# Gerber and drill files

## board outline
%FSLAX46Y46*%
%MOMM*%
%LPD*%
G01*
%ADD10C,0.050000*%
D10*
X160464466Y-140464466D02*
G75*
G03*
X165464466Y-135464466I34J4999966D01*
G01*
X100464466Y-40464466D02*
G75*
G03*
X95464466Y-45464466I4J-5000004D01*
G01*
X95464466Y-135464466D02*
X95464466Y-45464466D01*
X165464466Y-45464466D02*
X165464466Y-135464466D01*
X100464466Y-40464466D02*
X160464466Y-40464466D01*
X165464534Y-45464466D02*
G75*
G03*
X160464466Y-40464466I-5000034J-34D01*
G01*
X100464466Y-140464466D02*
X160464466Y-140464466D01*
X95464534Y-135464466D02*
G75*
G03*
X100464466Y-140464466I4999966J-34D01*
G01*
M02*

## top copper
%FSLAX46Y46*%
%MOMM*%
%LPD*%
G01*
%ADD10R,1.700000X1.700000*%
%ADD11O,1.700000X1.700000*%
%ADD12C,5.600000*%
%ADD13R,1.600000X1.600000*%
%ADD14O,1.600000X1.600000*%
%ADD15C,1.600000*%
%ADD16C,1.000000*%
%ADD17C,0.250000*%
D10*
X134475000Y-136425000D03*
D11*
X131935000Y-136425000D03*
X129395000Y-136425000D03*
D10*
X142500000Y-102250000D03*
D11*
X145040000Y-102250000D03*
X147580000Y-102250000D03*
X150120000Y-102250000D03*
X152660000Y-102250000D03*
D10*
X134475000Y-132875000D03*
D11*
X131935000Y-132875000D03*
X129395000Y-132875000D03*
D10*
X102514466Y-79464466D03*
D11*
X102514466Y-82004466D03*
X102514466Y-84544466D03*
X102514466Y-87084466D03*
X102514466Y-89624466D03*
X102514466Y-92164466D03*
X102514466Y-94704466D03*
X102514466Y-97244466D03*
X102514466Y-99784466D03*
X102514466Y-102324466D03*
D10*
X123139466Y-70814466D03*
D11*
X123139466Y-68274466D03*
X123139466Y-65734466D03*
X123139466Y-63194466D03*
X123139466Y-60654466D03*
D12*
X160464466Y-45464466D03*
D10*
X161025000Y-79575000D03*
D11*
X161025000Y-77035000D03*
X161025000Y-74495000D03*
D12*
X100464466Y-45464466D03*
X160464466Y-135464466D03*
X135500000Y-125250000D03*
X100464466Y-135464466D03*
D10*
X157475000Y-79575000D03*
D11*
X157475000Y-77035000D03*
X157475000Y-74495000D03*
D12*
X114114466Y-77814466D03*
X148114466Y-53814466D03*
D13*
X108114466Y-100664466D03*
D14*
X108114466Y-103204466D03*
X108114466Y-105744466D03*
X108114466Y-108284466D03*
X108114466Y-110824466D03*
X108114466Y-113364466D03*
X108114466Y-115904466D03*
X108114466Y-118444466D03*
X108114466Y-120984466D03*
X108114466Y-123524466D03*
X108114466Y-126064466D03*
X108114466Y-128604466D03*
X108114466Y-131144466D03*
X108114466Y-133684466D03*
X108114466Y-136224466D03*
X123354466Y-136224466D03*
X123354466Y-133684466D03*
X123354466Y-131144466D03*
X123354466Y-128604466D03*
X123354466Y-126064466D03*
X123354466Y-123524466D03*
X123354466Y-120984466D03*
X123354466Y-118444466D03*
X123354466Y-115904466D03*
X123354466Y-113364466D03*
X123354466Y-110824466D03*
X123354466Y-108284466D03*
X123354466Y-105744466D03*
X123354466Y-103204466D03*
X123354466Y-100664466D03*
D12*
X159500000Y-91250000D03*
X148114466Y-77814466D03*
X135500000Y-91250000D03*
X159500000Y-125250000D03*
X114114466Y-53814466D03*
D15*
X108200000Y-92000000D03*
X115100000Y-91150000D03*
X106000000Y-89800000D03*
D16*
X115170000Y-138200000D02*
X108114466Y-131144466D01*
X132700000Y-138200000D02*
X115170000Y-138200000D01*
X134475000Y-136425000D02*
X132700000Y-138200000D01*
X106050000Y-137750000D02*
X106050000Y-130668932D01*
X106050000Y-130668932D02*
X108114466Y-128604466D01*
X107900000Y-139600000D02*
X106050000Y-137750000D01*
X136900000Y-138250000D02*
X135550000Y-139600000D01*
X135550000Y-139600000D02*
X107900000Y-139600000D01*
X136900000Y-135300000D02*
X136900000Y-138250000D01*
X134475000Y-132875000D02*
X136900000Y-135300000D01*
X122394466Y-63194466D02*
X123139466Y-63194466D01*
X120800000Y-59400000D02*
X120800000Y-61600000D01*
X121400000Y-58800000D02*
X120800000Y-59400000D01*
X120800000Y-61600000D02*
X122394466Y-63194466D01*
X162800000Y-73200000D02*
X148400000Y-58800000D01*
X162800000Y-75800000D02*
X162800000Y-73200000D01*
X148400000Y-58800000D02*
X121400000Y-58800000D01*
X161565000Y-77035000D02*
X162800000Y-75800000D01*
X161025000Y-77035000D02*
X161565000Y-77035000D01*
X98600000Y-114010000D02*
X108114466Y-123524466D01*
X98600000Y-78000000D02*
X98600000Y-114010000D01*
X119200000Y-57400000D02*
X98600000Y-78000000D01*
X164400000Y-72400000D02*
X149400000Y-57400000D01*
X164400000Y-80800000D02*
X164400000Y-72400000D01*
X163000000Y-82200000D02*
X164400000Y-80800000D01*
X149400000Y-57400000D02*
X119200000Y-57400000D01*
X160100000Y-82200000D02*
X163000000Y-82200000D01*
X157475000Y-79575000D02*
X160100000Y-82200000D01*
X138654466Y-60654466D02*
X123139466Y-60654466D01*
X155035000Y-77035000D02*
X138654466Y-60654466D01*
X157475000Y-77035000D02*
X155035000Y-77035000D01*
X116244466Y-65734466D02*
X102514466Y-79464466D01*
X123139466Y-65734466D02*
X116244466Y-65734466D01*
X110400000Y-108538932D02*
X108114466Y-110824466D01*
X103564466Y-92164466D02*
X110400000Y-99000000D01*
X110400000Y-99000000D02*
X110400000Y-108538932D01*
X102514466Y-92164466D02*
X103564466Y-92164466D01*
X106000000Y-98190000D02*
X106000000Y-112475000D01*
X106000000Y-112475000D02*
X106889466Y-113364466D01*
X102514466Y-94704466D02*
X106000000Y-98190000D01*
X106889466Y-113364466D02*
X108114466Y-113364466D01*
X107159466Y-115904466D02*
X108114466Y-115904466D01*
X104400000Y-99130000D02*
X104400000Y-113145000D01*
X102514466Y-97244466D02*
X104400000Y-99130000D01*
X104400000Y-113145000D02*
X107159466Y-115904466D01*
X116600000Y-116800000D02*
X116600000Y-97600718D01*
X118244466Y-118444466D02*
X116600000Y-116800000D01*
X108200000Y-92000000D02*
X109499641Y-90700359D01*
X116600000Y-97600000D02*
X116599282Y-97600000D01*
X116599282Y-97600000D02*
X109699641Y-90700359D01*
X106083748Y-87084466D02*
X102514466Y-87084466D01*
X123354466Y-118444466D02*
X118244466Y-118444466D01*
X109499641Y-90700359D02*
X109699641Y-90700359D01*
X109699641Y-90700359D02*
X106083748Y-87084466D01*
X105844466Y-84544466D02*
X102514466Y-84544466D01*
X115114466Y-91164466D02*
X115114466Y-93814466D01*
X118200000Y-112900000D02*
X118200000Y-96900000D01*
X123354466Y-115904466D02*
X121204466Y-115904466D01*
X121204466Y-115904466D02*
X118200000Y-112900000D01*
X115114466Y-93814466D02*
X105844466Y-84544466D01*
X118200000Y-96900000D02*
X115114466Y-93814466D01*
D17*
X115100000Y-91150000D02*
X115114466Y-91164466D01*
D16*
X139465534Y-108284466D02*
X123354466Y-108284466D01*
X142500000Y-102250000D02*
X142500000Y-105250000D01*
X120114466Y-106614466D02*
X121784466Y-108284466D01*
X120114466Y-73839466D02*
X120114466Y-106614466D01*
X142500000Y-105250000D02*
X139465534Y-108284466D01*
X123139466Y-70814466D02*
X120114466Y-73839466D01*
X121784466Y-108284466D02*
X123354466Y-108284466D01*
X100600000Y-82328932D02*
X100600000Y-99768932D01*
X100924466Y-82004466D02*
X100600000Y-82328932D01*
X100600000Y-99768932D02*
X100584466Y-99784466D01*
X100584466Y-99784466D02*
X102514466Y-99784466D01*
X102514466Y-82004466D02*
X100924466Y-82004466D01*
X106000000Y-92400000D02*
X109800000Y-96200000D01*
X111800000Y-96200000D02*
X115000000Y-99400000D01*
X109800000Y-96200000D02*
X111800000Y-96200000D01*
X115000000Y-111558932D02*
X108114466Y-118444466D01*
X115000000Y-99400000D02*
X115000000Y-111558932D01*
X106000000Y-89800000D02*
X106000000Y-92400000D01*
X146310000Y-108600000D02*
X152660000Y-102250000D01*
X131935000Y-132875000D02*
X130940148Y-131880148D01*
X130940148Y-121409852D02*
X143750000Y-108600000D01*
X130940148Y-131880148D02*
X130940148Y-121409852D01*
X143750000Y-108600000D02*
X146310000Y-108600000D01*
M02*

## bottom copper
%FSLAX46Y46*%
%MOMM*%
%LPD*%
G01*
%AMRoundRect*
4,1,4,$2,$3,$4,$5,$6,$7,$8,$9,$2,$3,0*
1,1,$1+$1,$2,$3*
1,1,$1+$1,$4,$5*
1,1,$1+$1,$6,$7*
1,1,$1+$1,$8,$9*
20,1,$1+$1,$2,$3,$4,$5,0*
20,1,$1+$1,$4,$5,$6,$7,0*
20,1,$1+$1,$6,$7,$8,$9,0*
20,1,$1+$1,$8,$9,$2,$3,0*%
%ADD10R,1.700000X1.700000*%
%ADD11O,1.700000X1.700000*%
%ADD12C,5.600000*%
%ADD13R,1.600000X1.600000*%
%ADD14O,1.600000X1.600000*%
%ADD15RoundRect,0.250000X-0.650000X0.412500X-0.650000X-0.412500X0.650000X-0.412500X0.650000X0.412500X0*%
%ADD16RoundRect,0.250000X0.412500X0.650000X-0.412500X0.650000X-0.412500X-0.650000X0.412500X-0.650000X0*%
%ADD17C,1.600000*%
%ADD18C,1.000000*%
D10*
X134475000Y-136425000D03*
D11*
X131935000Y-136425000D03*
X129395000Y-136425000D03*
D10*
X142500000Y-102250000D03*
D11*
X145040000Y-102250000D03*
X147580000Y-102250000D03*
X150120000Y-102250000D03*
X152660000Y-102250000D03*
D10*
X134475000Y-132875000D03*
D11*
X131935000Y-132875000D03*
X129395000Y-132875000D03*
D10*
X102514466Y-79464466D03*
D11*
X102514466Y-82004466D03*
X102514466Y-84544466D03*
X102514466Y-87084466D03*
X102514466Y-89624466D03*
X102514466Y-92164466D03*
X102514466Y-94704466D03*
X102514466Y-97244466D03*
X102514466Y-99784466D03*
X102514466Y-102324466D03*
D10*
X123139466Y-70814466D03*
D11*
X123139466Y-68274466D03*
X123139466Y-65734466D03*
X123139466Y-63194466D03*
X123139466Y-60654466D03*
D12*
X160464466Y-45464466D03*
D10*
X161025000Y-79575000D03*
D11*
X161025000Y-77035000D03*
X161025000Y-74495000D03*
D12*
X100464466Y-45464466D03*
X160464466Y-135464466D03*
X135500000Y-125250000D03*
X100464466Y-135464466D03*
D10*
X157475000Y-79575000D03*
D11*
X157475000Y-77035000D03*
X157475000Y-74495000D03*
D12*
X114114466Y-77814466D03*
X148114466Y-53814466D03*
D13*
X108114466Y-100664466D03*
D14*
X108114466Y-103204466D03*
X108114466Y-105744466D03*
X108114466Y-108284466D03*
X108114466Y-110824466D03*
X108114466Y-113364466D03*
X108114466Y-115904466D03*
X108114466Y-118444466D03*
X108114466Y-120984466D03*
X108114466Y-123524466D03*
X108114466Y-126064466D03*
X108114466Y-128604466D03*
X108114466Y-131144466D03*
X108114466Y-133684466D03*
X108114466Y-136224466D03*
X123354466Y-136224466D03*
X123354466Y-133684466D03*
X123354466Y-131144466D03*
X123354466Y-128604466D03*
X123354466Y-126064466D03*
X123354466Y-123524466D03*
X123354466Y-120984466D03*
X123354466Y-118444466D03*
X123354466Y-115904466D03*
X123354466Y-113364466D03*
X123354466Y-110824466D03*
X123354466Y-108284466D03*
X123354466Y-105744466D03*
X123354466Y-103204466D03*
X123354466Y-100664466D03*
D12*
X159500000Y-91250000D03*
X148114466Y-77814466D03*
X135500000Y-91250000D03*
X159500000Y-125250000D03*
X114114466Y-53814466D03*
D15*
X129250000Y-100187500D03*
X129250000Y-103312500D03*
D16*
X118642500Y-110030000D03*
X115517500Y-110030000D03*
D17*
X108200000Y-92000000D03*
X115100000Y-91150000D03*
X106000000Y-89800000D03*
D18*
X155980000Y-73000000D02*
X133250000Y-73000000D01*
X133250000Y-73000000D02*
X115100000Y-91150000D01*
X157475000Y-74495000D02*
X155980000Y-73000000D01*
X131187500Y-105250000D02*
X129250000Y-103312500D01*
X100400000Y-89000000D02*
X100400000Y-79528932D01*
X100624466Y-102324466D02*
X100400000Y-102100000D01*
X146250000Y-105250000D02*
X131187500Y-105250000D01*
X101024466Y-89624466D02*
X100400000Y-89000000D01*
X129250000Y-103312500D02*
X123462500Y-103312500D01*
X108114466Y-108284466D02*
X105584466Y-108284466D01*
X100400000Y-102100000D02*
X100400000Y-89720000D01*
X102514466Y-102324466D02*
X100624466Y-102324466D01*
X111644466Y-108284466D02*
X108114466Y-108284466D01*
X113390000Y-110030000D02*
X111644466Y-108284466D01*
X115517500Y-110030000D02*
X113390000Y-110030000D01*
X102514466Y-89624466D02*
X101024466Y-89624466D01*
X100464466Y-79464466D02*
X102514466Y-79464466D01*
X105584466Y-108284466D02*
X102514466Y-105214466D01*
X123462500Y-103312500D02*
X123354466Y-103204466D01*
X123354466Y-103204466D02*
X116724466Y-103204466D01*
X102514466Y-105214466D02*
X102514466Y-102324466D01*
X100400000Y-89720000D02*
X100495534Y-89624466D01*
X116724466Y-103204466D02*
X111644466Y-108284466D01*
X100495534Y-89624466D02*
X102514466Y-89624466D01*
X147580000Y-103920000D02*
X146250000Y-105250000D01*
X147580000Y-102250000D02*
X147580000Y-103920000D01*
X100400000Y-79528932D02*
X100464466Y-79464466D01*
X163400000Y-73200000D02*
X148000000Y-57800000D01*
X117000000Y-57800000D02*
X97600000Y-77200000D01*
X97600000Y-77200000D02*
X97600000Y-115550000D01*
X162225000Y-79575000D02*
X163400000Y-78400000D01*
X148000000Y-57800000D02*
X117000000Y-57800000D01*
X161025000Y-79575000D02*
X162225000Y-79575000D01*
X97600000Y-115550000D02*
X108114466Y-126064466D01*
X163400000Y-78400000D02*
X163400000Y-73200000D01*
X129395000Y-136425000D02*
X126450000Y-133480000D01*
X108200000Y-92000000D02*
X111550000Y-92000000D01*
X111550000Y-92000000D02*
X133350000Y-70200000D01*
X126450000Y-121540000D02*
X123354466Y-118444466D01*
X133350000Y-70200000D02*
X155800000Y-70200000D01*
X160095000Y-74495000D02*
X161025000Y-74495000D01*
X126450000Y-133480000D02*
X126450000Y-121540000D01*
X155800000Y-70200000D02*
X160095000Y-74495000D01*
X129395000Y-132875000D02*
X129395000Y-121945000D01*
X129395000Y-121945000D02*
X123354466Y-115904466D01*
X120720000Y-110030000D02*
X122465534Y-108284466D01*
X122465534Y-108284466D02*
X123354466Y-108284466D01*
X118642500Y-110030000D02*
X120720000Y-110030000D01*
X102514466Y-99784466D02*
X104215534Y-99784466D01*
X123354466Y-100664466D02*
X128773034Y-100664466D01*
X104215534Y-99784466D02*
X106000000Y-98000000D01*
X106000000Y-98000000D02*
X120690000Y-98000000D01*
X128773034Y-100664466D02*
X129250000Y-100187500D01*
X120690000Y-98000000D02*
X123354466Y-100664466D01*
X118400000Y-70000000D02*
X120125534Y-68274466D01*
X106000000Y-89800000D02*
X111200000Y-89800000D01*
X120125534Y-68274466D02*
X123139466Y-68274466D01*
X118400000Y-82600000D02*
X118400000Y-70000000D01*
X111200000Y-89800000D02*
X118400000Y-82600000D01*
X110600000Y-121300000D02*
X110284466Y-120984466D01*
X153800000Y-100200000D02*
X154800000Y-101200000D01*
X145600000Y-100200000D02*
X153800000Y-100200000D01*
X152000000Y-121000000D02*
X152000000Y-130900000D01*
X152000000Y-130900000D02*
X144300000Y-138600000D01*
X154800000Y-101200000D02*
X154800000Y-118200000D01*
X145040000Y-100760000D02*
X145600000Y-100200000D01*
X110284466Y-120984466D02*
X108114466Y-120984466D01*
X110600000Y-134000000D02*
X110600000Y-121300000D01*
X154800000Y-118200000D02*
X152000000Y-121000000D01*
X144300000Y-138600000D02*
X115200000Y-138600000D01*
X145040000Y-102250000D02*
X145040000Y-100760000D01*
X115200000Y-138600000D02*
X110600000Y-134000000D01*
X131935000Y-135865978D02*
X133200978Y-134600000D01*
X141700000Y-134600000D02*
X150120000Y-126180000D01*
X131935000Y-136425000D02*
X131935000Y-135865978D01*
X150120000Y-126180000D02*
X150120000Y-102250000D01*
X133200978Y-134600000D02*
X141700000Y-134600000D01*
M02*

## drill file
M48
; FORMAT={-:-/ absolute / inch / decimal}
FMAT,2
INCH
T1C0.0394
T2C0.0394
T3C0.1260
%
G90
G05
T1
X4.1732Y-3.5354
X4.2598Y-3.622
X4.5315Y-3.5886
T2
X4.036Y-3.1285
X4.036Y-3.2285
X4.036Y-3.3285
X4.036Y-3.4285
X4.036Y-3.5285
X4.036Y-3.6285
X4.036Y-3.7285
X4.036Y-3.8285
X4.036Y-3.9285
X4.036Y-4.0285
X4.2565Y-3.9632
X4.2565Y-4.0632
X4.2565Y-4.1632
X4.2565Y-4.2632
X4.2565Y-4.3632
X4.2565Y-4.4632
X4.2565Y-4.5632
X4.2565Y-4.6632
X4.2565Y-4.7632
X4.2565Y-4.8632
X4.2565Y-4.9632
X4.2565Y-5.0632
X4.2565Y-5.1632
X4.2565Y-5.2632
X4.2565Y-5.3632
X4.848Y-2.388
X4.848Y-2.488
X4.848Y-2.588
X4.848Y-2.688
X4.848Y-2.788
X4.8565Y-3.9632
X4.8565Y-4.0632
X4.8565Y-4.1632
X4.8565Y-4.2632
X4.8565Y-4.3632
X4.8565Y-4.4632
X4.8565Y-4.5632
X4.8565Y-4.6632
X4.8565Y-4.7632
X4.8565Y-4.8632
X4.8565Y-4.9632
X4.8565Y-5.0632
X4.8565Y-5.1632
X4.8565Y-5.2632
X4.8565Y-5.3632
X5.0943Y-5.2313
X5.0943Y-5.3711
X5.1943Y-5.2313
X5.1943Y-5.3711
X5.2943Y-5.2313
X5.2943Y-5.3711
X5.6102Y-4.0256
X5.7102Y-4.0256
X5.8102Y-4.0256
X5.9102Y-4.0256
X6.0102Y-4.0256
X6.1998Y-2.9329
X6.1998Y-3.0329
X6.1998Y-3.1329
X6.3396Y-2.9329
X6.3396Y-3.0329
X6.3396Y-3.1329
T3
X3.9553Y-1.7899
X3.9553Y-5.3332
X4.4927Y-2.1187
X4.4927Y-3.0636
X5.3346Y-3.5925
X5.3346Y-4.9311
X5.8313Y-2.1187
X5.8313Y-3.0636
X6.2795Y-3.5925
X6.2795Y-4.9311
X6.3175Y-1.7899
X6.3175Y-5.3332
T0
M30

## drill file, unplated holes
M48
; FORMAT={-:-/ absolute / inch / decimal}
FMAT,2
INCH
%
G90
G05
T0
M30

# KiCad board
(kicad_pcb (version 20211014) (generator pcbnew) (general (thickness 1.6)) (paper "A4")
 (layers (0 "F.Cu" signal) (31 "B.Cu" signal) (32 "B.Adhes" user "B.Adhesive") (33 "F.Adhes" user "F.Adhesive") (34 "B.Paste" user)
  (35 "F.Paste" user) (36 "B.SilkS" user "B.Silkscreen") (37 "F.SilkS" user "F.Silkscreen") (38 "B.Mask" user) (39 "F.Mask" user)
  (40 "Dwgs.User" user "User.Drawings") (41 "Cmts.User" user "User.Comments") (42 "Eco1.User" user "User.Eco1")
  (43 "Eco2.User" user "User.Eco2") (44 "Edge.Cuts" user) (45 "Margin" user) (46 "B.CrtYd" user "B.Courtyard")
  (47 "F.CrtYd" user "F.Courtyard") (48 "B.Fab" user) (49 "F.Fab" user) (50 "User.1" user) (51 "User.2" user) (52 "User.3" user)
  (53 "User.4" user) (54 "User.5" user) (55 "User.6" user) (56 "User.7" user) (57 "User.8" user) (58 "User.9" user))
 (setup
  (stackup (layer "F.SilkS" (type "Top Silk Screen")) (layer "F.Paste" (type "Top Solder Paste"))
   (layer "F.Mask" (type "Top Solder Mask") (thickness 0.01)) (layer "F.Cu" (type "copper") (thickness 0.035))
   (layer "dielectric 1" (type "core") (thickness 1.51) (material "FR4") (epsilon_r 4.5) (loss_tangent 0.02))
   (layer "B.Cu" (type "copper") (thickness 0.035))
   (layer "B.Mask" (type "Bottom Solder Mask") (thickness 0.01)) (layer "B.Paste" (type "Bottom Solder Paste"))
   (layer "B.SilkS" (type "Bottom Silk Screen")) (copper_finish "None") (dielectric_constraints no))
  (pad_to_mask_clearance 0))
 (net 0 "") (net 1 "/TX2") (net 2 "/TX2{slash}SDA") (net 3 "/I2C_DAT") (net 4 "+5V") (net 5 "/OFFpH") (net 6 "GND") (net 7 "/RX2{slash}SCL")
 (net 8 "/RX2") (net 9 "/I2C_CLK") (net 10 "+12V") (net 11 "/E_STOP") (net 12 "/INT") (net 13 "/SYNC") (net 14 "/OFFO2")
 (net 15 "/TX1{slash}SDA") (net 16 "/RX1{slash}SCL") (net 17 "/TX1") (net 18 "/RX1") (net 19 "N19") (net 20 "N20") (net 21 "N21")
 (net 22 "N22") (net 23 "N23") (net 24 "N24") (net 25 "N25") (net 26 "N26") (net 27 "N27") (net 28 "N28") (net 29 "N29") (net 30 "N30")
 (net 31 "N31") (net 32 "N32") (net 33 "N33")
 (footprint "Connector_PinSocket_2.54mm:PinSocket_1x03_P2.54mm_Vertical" (layer "F.Cu") (at 134.475 136.425 -90)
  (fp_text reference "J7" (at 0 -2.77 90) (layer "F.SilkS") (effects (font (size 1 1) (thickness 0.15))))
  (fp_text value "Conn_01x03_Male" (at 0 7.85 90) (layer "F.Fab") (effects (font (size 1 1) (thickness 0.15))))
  (pad "1" thru_hole rect (at 0 0 270) (size 1.7 1.7) (drill 1) (layers *.Cu *.Mask) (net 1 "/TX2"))
  (pad "2" thru_hole oval (at 0 2.54 270) (size 1.7 1.7) (drill 1) (layers *.Cu *.Mask) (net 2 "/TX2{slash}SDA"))
  (pad "3" thru_hole oval (at 0 5.08 270) (size 1.7 1.7) (drill 1) (layers *.Cu *.Mask) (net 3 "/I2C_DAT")))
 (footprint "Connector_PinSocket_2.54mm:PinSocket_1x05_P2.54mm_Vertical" (layer "F.Cu") (at 142.5 102.25 90)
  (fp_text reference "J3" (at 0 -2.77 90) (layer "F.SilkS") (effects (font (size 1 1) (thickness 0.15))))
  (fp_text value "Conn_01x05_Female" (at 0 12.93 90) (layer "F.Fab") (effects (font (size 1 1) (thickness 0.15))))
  (pad "1" thru_hole rect (at 0 0 90) (size 1.7 1.7) (drill 1) (layers *.Cu *.Mask) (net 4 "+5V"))
  (pad "2" thru_hole oval (at 0 2.54 90) (size 1.7 1.7) (drill 1) (layers *.Cu *.Mask) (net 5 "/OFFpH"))
  (pad "3" thru_hole oval (at 0 5.08 90) (size 1.7 1.7) (drill 1) (layers *.Cu *.Mask) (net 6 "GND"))
  (pad "4" thru_hole oval (at 0 7.62 90) (size 1.7 1.7) (drill 1) (layers *.Cu *.Mask) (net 2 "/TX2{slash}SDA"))
  (pad "5" thru_hole oval (at 0 10.16 90) (size 1.7 1.7) (drill 1) (layers *.Cu *.Mask) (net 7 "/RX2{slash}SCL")))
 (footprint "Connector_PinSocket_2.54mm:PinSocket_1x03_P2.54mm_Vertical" (layer "F.Cu") (at 134.475 132.875 -90)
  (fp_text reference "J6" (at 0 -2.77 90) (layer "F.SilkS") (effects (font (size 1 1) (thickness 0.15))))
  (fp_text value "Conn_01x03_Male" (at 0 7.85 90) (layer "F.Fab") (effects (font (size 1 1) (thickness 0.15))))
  (pad "1" thru_hole rect (at 0 0 270) (size 1.7 1.7) (drill 1) (layers *.Cu *.Mask) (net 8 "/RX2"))
  (pad "2" thru_hole oval (at 0 2.54 270) (size 1.7 1.7) (drill 1) (layers *.Cu *.Mask) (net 7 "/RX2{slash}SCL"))
  (pad "3" thru_hole oval (at 0 5.08 270) (size 1.7 1.7) (drill 1) (layers *.Cu *.Mask) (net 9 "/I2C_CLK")))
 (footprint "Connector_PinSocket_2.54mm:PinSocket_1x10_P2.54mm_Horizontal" (layer "F.Cu") (at 102.514466 79.464466)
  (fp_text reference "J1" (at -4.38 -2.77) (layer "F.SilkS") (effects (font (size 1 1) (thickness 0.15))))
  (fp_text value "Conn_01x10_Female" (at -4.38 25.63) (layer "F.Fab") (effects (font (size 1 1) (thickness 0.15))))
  (pad "1" thru_hole rect (at 0 0) (size 1.7 1.7) (drill 1) (layers *.Cu *.Mask) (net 6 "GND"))
  (pad "2" thru_hole oval (at 0 2.54) (size 1.7 1.7) (drill 1) (layers *.Cu *.Mask) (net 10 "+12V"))
  (pad "3" thru_hole oval (at 0 5.08) (size 1.7 1.7) (drill 1) (layers *.Cu *.Mask) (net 9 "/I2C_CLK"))
  (pad "4" thru_hole oval (at 0 7.62) (size 1.7 1.7) (drill 1) (layers *.Cu *.Mask) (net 3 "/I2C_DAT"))
  (pad "5" thru_hole oval (at 0 10.16) (size 1.7 1.7) (drill 1) (layers *.Cu *.Mask) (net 6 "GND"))
  (pad "6" thru_hole oval (at 0 12.7) (size 1.7 1.7) (drill 1) (layers *.Cu *.Mask) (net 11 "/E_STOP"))
  (pad "7" thru_hole oval (at 0 15.24) (size 1.7 1.7) (drill 1) (layers *.Cu *.Mask) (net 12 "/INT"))
  (pad "8" thru_hole oval (at 0 17.78) (size 1.7 1.7) (drill 1) (layers *.Cu *.Mask) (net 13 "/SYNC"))
  (pad "9" thru_hole oval (at 0 20.32) (size 1.7 1.7) (drill 1) (layers *.Cu *.Mask) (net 10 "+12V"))
  (pad "10" thru_hole oval (at 0 22.86) (size 1.7 1.7) (drill 1) (layers *.Cu *.Mask) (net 6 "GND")))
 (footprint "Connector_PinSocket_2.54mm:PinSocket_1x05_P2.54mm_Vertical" (layer "F.Cu") (at 123.139466 70.814466 180)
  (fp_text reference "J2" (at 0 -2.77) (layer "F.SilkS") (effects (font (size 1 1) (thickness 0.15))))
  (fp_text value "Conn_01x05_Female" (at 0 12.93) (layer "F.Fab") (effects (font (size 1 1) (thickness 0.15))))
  (pad "1" thru_hole rect (at 0 0 180) (size 1.7 1.7) (drill 1) (layers *.Cu *.Mask) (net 4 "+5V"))
  (pad "2" thru_hole oval (at 0 2.54 180) (size 1.7 1.7) (drill 1) (layers *.Cu *.Mask) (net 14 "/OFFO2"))
  (pad "3" thru_hole oval (at 0 5.08 180) (size 1.7 1.7) (drill 1) (layers *.Cu *.Mask) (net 6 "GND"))
  (pad "4" thru_hole oval (at 0 7.62 180) (size 1.7 1.7) (drill 1) (layers *.Cu *.Mask) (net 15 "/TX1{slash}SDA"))
  (pad "5" thru_hole oval (at 0 10.16 180) (size 1.7 1.7) (drill 1) (layers *.Cu *.Mask) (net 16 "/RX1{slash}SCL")))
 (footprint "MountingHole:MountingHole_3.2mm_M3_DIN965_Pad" (layer "F.Cu") (at 160.464466 45.464466)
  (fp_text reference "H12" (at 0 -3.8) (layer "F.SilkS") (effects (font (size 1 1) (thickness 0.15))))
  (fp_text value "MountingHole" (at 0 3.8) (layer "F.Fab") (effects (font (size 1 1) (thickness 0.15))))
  (pad "1" thru_hole circle (at 0 0) (size 5.6 5.6) (drill 3.2) (layers *.Cu *.Mask)))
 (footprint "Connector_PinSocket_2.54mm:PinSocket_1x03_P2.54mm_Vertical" (layer "F.Cu") (at 161.025 79.575 180)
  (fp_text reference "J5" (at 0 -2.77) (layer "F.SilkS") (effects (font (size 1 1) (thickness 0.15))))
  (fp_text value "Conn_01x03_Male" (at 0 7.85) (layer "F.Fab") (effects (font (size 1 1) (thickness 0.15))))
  (pad "1" thru_hole rect (at 0 0 180) (size 1.7 1.7) (drill 1) (layers *.Cu *.Mask) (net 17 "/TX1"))
  (pad "2" thru_hole oval (at 0 2.54 180) (size 1.7 1.7) (drill 1) (layers *.Cu *.Mask) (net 15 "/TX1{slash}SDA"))
  (pad "3" thru_hole oval (at 0 5.08 180) (size 1.7 1.7) (drill 1) (layers *.Cu *.Mask) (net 3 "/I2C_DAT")))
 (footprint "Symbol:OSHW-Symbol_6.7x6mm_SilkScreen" (layer "F.Cu") (at 109.515 44.979 180)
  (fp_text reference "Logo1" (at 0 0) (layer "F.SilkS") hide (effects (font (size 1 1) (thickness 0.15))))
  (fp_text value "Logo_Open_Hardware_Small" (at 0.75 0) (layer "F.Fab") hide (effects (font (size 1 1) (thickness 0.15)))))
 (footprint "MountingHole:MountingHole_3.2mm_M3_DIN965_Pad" (layer "F.Cu") (at 100.464466 45.464466)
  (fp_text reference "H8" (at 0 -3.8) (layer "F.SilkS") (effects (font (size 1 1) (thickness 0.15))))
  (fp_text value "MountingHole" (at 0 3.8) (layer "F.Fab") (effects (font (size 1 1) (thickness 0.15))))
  (pad "1" thru_hole circle (at 0 0) (size 5.6 5.6) (drill 3.2) (layers *.Cu *.Mask)))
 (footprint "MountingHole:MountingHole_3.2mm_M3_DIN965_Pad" (layer "F.Cu") (at 160.464466 135.464466)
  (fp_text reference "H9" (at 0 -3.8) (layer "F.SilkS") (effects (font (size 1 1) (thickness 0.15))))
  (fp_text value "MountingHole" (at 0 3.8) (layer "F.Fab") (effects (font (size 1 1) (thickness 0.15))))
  (pad "1" thru_hole circle (at 0 0) (size 5.6 5.6) (drill 3.2) (layers *.Cu *.Mask)))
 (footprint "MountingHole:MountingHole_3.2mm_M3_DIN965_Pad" (layer "F.Cu") (at 135.5 125.25 90)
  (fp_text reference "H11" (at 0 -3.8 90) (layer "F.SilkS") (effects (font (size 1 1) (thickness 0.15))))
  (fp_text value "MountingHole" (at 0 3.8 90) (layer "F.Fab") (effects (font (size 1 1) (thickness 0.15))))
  (pad "1" thru_hole circle (at 0 0 90) (size 5.6 5.6) (drill 3.2) (layers *.Cu *.Mask)))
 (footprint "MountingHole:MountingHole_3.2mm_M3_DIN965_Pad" (layer "F.Cu") (at 100.464466 135.464466)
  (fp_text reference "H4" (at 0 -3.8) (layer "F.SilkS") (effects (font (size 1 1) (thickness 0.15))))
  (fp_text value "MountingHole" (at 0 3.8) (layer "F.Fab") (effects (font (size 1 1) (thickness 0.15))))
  (pad "1" thru_hole circle (at 0 0) (size 5.6 5.6) (drill 3.2) (layers *.Cu *.Mask)))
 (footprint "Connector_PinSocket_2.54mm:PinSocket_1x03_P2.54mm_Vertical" (layer "F.Cu") (at 157.475 79.575 180)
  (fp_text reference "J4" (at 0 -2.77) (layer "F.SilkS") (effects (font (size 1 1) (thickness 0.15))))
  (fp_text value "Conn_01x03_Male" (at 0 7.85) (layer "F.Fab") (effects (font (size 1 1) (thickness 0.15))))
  (pad "1" thru_hole rect (at 0 0 180) (size 1.7 1.7) (drill 1) (layers *.Cu *.Mask) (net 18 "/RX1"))
  (pad "2" thru_hole oval (at 0 2.54 180) (size 1.7 1.7) (drill 1) (layers *.Cu *.Mask) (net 16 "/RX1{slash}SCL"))
  (pad "3" thru_hole oval (at 0 5.08 180) (size 1.7 1.7) (drill 1) (layers *.Cu *.Mask) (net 9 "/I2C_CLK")))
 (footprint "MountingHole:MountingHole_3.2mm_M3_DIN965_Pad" (layer "F.Cu") (at 114.114466 77.814466)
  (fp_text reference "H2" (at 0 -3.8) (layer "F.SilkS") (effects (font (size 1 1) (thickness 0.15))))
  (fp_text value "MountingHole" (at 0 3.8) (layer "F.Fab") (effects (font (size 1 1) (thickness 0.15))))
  (pad "1" thru_hole circle (at 0 0) (size 5.6 5.6) (drill 3.2) (layers *.Cu *.Mask)))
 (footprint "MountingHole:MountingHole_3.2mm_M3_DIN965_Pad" (layer "F.Cu") (at 148.114466 53.814466)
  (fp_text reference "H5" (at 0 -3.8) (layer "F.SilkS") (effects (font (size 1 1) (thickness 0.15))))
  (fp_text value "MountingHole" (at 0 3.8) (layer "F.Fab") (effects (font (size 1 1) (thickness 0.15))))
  (pad "1" thru_hole circle (at 0 0) (size 5.6 5.6) (drill 3.2) (layers *.Cu *.Mask)))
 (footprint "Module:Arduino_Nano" (layer "F.Cu") (at 108.114466 100.664466)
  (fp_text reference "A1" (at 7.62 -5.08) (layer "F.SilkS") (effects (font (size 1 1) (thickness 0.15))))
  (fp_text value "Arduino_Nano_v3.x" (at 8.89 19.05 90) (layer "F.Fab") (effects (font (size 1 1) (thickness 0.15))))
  (pad "1" thru_hole rect (at 0 0) (size 1.6 1.6) (drill 1) (layers *.Cu *.Mask) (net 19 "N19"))
  (pad "2" thru_hole oval (at 0 2.54) (size 1.6 1.6) (drill 1) (layers *.Cu *.Mask) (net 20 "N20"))
  (pad "3" thru_hole oval (at 0 5.08) (size 1.6 1.6) (drill 1) (layers *.Cu *.Mask) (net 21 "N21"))
  (pad "4" thru_hole oval (at 0 7.62) (size 1.6 1.6) (drill 1) (layers *.Cu *.Mask) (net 6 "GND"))
  (pad "5" thru_hole oval (at 0 10.16) (size 1.6 1.6) (drill 1) (layers *.Cu *.Mask) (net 11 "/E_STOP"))
  (pad "6" thru_hole oval (at 0 12.7) (size 1.6 1.6) (drill 1) (layers *.Cu *.Mask) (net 12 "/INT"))
  (pad "7" thru_hole oval (at 0 15.24) (size 1.6 1.6) (drill 1) (layers *.Cu *.Mask) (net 13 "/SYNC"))
  (pad "8" thru_hole oval (at 0 17.78) (size 1.6 1.6) (drill 1) (layers *.Cu *.Mask) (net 14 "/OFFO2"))
  (pad "9" thru_hole oval (at 0 20.32) (size 1.6 1.6) (drill 1) (layers *.Cu *.Mask) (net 5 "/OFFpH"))
  (pad "10" thru_hole oval (at 0 22.86) (size 1.6 1.6) (drill 1) (layers *.Cu *.Mask) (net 18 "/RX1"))
  (pad "11" thru_hole oval (at 0 25.4) (size 1.6 1.6) (drill 1) (layers *.Cu *.Mask) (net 17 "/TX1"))
  (pad "12" thru_hole oval (at 0 27.94) (size 1.6 1.6) (drill 1) (layers *.Cu *.Mask) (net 8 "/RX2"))
  (pad "13" thru_hole oval (at 0 30.48) (size 1.6 1.6) (drill 1) (layers *.Cu *.Mask) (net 1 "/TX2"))
  (pad "14" thru_hole oval (at 0 33.02) (size 1.6 1.6) (drill 1) (layers *.Cu *.Mask) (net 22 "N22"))
  (pad "15" thru_hole oval (at 0 35.56) (size 1.6 1.6) (drill 1) (layers *.Cu *.Mask) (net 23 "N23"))
  (pad "16" thru_hole oval (at 15.24 35.56) (size 1.6 1.6) (drill 1) (layers *.Cu *.Mask) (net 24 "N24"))
  (pad "17" thru_hole oval (at 15.24 33.02) (size 1.6 1.6) (drill 1) (layers *.Cu *.Mask) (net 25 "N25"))
  (pad "18" thru_hole oval (at 15.24 30.48) (size 1.6 1.6) (drill 1) (layers *.Cu *.Mask) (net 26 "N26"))
  (pad "19" thru_hole oval (at 15.24 27.94) (size 1.6 1.6) (drill 1) (layers *.Cu *.Mask) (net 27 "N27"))
  (pad "20" thru_hole oval (at 15.24 25.4) (size 1.6 1.6) (drill 1) (layers *.Cu *.Mask) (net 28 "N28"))
  (pad "21" thru_hole oval (at 15.24 22.86) (size 1.6 1.6) (drill 1) (layers *.Cu *.Mask) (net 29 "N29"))
  (pad "22" thru_hole oval (at 15.24 20.32) (size 1.6 1.6) (drill 1) (layers *.Cu *.Mask) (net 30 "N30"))
  (pad "23" thru_hole oval (at 15.24 17.78) (size 1.6 1.6) (drill 1) (layers *.Cu *.Mask) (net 3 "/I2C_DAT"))
  (pad "24" thru_hole oval (at 15.24 15.24) (size 1.6 1.6) (drill 1) (layers *.Cu *.Mask) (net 9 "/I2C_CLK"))
  (pad "25" thru_hole oval (at 15.24 12.7) (size 1.6 1.6) (drill 1) (layers *.Cu *.Mask) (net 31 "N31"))
  (pad "26" thru_hole oval (at 15.24 10.16) (size 1.6 1.6) (drill 1) (layers *.Cu *.Mask) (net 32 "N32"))
  (pad "27" thru_hole oval (at 15.24 7.62) (size 1.6 1.6) (drill 1) (layers *.Cu *.Mask) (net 4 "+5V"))
  (pad "28" thru_hole oval (at 15.24 5.08) (size 1.6 1.6) (drill 1) (layers *.Cu *.Mask) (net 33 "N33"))
  (pad "29" thru_hole oval (at 15.24 2.54) (size 1.6 1.6) (drill 1) (layers *.Cu *.Mask) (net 6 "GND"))
  (pad "30" thru_hole oval (at 15.24 0) (size 1.6 1.6) (drill 1) (layers *.Cu *.Mask) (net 10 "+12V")))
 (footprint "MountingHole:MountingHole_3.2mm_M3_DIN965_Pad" (layer "F.Cu") (at 159.5 91.25 90)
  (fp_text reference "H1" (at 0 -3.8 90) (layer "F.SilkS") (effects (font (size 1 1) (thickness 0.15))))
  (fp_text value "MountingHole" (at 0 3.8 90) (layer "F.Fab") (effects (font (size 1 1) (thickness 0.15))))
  (pad "1" thru_hole circle (at 0 0 90) (size 5.6 5.6) (drill 3.2) (layers *.Cu *.Mask)))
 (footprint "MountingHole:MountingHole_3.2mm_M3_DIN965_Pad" (layer "F.Cu") (at 148.114466 77.814466)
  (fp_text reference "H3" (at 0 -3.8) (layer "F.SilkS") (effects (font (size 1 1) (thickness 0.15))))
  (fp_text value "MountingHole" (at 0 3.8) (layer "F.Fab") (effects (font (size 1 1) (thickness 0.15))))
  (pad "1" thru_hole circle (at 0 0) (size 5.6 5.6) (drill 3.2) (layers *.Cu *.Mask)))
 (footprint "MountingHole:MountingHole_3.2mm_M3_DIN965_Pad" (layer "F.Cu") (at 135.5 91.25 90)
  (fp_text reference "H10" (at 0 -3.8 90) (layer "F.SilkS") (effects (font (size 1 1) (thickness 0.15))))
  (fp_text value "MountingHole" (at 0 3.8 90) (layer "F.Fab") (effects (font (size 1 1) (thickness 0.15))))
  (pad "1" thru_hole circle (at 0 0 90) (size 5.6 5.6) (drill 3.2) (layers *.Cu *.Mask)))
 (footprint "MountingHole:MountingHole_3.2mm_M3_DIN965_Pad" (layer "F.Cu") (at 159.5 125.25 90)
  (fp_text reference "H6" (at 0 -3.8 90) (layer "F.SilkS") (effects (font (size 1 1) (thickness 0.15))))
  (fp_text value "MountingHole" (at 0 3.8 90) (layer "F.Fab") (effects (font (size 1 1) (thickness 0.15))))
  (pad "1" thru_hole circle (at 0 0 90) (size 5.6 5.6) (drill 3.2) (layers *.Cu *.Mask)))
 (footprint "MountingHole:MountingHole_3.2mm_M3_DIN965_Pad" (layer "F.Cu") (at 114.114466 53.814466)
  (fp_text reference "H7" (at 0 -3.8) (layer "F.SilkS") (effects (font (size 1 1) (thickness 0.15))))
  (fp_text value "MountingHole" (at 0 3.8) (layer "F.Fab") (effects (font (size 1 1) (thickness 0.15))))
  (pad "1" thru_hole circle (at 0 0) (size 5.6 5.6) (drill 3.2) (layers *.Cu *.Mask)))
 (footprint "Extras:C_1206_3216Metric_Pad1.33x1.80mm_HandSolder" (layer "B.Cu") (at 129.25 101.75 -90)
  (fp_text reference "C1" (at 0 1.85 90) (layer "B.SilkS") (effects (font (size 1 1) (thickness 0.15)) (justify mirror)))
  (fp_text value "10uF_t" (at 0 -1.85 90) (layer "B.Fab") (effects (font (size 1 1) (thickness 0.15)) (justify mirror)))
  (pad "1" smd roundrect (at -1.5625 0 270) (size 1.325 1.8) (layers "B.Cu" "B.Paste" "B.Mask") (roundrect_rratio 0.1886792453)
   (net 10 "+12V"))
  (pad "2" smd roundrect (at 1.5625 0 270) (size 1.325 1.8) (layers "B.Cu" "B.Paste" "B.Mask") (roundrect_rratio 0.1886792453) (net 6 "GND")))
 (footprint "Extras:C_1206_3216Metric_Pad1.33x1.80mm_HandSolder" (layer "B.Cu") (at 117.08 110.03 180)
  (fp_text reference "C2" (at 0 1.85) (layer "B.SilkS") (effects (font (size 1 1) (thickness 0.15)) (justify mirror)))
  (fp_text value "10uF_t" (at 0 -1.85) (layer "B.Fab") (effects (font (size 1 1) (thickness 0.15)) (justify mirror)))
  (pad "1" smd roundrect (at -1.5625 0 180) (size 1.325 1.8) (layers "B.Cu" "B.Paste" "B.Mask") (roundrect_rratio 0.1886792453)
   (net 4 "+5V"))
  (pad "2" smd roundrect (at 1.5625 0 180) (size 1.325 1.8) (layers "B.Cu" "B.Paste" "B.Mask") (roundrect_rratio 0.1886792453) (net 6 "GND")))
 (gr_arc (start 165.464466 135.464466) (mid 164 139) (end 160.464466 140.464466) (layer "Edge.Cuts") (width 0.05))
 (gr_arc (start 95.464466 45.464466) (mid 96.928932 41.928932) (end 100.464466 40.464466) (layer "Edge.Cuts") (width 0.05))
 (gr_line (start 95.464466 135.464466) (end 95.464466 45.464466) (layer "Edge.Cuts") (width 0.05))
 (gr_line (start 165.464466 45.464466) (end 165.464466 135.464466) (layer "Edge.Cuts") (width 0.05))
 (gr_line (start 100.464466 40.464466) (end 160.464466 40.464466) (layer "Edge.Cuts") (width 0.05))
 (gr_arc (start 160.464466 40.464466) (mid 164 41.928932) (end 165.464466 45.464466) (layer "Edge.Cuts") (width 0.05))
 (gr_line (start 100.464466 140.464466) (end 160.464466 140.464466) (layer "Edge.Cuts") (width 0.05))
 (gr_arc (start 100.464466 140.464466) (mid 96.928932 139) (end 95.464466 135.464466) (layer "Edge.Cuts") (width 0.05))
 (segment (start 116.244466 65.734466) (end 102.514466 79.464466) (width 1) (layer "F.Cu") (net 6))
 (segment (start 123.139466 65.734466) (end 116.244466 65.734466) (width 1) (layer "F.Cu") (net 6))
 (segment (start 131.1875 105.25) (end 129.25 103.3125) (width 1) (layer "B.Cu") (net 6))
 (segment (start 100.4 89) (end 100.4 79.528932) (width 1) (layer "B.Cu") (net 6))
 (segment (start 100.624466 102.324466) (end 100.4 102.1) (width 1) (layer "B.Cu") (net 6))
 (segment (start 146.25 105.25) (end 131.1875 105.25) (width 1) (layer "B.Cu") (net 6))
 (segment (start 101.024466 89.624466) (end 100.4 89) (width 1) (layer "B.Cu") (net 6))
 (segment (start 129.25 103.3125) (end 123.4625 103.3125) (width 1) (layer "B.Cu") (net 6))
 (segment (start 108.114466 108.284466) (end 105.584466 108.284466) (width 1) (layer "B.Cu") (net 6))
 (segment (start 100.4 102.1) (end 100.4 89.72) (width 1) (layer "B.Cu") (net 6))
 (segment (start 102.514466 102.324466) (end 100.624466 102.324466) (width 1) (layer "B.Cu") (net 6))
 (segment (start 111.644466 108.284466) (end 108.114466 108.284466) (width 1) (layer "B.Cu") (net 6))
 (segment (start 113.39 110.03) (end 111.644466 108.284466) (width 1) (layer "B.Cu") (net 6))
 (segment (start 115.5175 110.03) (end 113.39 110.03) (width 1) (layer "B.Cu") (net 6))
 (segment (start 102.514466 89.624466) (end 101.024466 89.624466) (width 1) (layer "B.Cu") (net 6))
 (segment (start 100.464466 79.464466) (end 102.514466 79.464466) (width 1) (layer "B.Cu") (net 6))
 (segment (start 105.584466 108.284466) (end 102.514466 105.214466) (width 1) (layer "B.Cu") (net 6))
 (segment (start 123.4625 103.3125) (end 123.354466 103.204466) (width 1) (layer "B.Cu") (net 6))
 (segment (start 123.354466 103.204466) (end 116.724466 103.204466) (width 1) (layer "B.Cu") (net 6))
 (segment (start 102.514466 105.214466) (end 102.514466 102.324466) (width 1) (layer "B.Cu") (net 6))
 (segment (start 100.4 89.72) (end 100.495534 89.624466) (width 1) (layer "B.Cu") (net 6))
 (segment (start 116.724466 103.204466) (end 111.644466 108.284466) (width 1) (layer "B.Cu") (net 6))
 (segment (start 100.495534 89.624466) (end 102.514466 89.624466) (width 1) (layer "B.Cu") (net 6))
 (segment (start 147.58 103.92) (end 146.25 105.25) (width 1) (layer "B.Cu") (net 6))
 (segment (start 147.58 102.25) (end 147.58 103.92) (width 1) (layer "B.Cu") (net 6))
 (segment (start 100.4 79.528932) (end 100.464466 79.464466) (width 1) (layer "B.Cu") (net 6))
 (segment (start 110.4 108.538932) (end 108.114466 110.824466) (width 1) (layer "F.Cu") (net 11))
 (segment (start 103.564466 92.164466) (end 110.4 99) (width 1) (layer "F.Cu") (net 11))
 (segment (start 110.4 99) (end 110.4 108.538932) (width 1) (layer "F.Cu") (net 11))
 (segment (start 102.514466 92.164466) (end 103.564466 92.164466) (width 1) (layer "F.Cu") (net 11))
 (segment (start 106 98.19) (end 106 112.475) (width 1) (layer "F.Cu") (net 12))
 (segment (start 106 112.475) (end 106.889466 113.364466) (width 1) (layer "F.Cu") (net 12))
 (segment (start 102.514466 94.704466) (end 106 98.19) (width 1) (layer "F.Cu") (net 12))
 (segment (start 106.889466 113.364466) (end 108.114466 113.364466) (width 1) (layer "F.Cu") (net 12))
 (segment (start 107.159466 115.904466) (end 108.114466 115.904466) (width 1) (layer "F.Cu") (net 13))
 (segment (start 104.4 99.13) (end 104.4 113.145) (width 1) (layer "F.Cu") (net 13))
 (segment (start 102.514466 97.244466) (end 104.4 99.13) (width 1) (layer "F.Cu") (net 13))
 (segment (start 104.4 113.145) (end 107.159466 115.904466) (width 1) (layer "F.Cu") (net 13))
 (segment (start 98.6 114.01) (end 108.114466 123.524466) (width 1) (layer "F.Cu") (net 18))
 (segment (start 164.4 72.4) (end 149.4 57.4) (width 1) (layer "F.Cu") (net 18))
 (segment (start 164.4 80.8) (end 164.4 72.4) (width 1) (layer "F.Cu") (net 18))
 (segment (start 119.2 57.4) (end 98.6 78) (width 1) (layer "F.Cu") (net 18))
 (segment (start 98.6 78) (end 98.6 114.01) (width 1) (layer "F.Cu") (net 18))
 (segment (start 149.4 57.4) (end 119.2 57.4) (width 1) (layer "F.Cu") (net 18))
 (segment (start 160.1 82.2) (end 163 82.2) (width 1) (layer "F.Cu") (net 18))
 (segment (start 163 82.2) (end 164.4 80.8) (width 1) (layer "F.Cu") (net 18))
 (segment (start 157.475 79.575) (end 160.1 82.2) (width 1) (layer "F.Cu") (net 18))
 (segment (start 163.4 73.2) (end 148 57.8) (width 1) (layer "B.Cu") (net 17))
 (segment (start 117 57.8) (end 97.6 77.2) (width 1) (layer "B.Cu") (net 17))
 (segment (start 97.6 77.2) (end 97.6 115.55) (width 1) (layer "B.Cu") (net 17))
 (segment (start 162.225 79.575) (end 163.4 78.4) (width 1) (layer "B.Cu") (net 17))
 (segment (start 148 57.8) (end 117 57.8) (width 1) (layer "B.Cu") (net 17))
 (segment (start 161.025 79.575) (end 162.225 79.575) (width 1) (layer "B.Cu") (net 17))
 (segment (start 97.6 115.55) (end 108.114466 126.064466) (width 1) (layer "B.Cu") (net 17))
 (segment (start 163.4 78.4) (end 163.4 73.2) (width 1) (layer "B.Cu") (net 17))
 (segment (start 107.9 139.6) (end 106.05 137.75) (width 1) (layer "F.Cu") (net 8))
 (segment (start 136.9 138.25) (end 135.55 139.6) (width 1) (layer "F.Cu") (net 8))
 (segment (start 135.55 139.6) (end 107.9 139.6) (width 1) (layer "F.Cu") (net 8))
 (segment (start 106.05 137.75) (end 106.05 130.668932) (width 1) (layer "F.Cu") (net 8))
 (segment (start 106.05 130.668932) (end 108.114466 128.604466) (width 1) (layer "F.Cu") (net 8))
 (segment (start 134.475 132.875) (end 136.9 135.3) (width 1) (layer "F.Cu") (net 8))
 (segment (start 136.9 135.3) (end 136.9 138.25) (width 1) (layer "F.Cu") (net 8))
 (segment (start 134.475 136.425) (end 132.7 138.2) (width 1) (layer "F.Cu") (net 1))
 (segment (start 132.7 138.2) (end 115.17 138.2) (width 1) (layer "F.Cu") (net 1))
 (segment (start 115.17 138.2) (end 108.114466 131.144466) (width 1) (layer "F.Cu") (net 1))
 (segment (start 116.6 116.8) (end 116.6 97.600718) (width 1) (layer "F.Cu") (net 3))
 (segment (start 118.244466 118.444466) (end 116.6 116.8) (width 1) (layer "F.Cu") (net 3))
 (segment (start 108.2 92) (end 109.499641 90.700359) (width 1) (layer "F.Cu") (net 3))
 (segment (start 116.6 97.6) (end 116.599282 97.6) (width 1) (layer "F.Cu") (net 3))
 (segment (start 116.599282 97.6) (end 109.699641 90.700359) (width 1) (layer "F.Cu") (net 3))
 (segment (start 106.083748 87.084466) (end 102.514466 87.084466) (width 1) (layer "F.Cu") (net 3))
 (segment (start 123.354466 118.444466) (end 118.244466 118.444466) (width 1) (layer "F.Cu") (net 3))
 (segment (start 109.499641 90.700359) (end 109.699641 90.700359) (width 1) (layer "F.Cu") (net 3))
 (segment (start 109.699641 90.700359) (end 106.083748 87.084466) (width 1) (layer "F.Cu") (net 3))
 (via (at 108.2 92) (size 1.6) (drill 1) (layers "F.Cu" "B.Cu") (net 3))
 (segment (start 129.395 136.425) (end 126.45 133.48) (width 1) (layer "B.Cu") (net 3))
 (segment (start 108.2 92) (end 111.55 92) (width 1) (layer "B.Cu") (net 3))
 (segment (start 111.55 92) (end 133.35 70.2) (width 1) (layer "B.Cu") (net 3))
 (segment (start 126.45 121.54) (end 123.354466 118.444466) (width 1) (layer "B.Cu") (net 3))
 (segment (start 133.35 70.2) (end 155.8 70.2) (width 1) (layer "B.Cu") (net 3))
 (segment (start 160.095 74.495) (end 161.025 74.495) (width 1) (layer "B.Cu") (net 3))
 (segment (start 126.45 133.48) (end 126.45 121.54) (width 1) (layer "B.Cu") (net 3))
 (segment (start 155.8 70.2) (end 160.095 74.495) (width 1) (layer "B.Cu") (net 3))
 (segment (start 105.844466 84.544466) (end 102.514466 84.544466) (width 1) (layer "F.Cu") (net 9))
 (segment (start 115.114466 91.164466) (end 115.114466 93.814466) (width 1) (layer "F.Cu") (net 9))
 (segment (start 118.2 112.9) (end 118.2 96.9) (width 1) (layer "F.Cu") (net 9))
 (segment (start 123.354466 115.904466) (end 121.204466 115.904466) (width 1) (layer "F.Cu") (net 9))
 (segment (start 121.204466 115.904466) (end 118.2 112.9) (width 1) (layer "F.Cu") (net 9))
 (segment (start 115.114466 93.814466) (end 105.844466 84.544466) (width 1) (layer "F.Cu") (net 9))
 (segment (start 118.2 96.9) (end 115.114466 93.814466) (width 1) (layer "F.Cu") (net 9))
 (segment (start 115.1 91.15) (end 115.114466 91.164466) (width 0.25) (layer "F.Cu") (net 9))
 (via (at 115.1 91.15) (size 1.6) (drill 1) (layers "F.Cu" "B.Cu") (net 9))
 (segment (start 133.25 73) (end 115.1 91.15) (width 1) (layer "B.Cu") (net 9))
 (segment (start 155.98 73) (end 133.25 73) (width 1) (layer "B.Cu") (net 9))
 (segment (start 129.395 132.875) (end 129.395 121.945) (width 1) (layer "B.Cu") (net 9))
 (segment (start 129.395 121.945) (end 123.354466 115.904466) (width 1) (layer "B.Cu") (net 9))
 (segment (start 157.475 74.495) (end 155.98 73) (width 1) (layer "B.Cu") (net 9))
 (segment (start 139.465534 108.284466) (end 123.354466 108.284466) (width 1) (layer "F.Cu") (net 4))
 (segment (start 142.5 102.25) (end 142.5 105.25) (width 1) (layer "F.Cu") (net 4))
 (segment (start 120.114466 106.614466) (end 121.784466 108.284466) (width 1) (layer "F.Cu") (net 4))
 (segment (start 120.114466 73.839466) (end 120.114466 106.614466) (width 1) (layer "F.Cu") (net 4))
 (segment (start 142.5 105.25) (end 139.465534 108.284466) (width 1) (layer "F.Cu") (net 4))
 (segment (start 123.139466 70.814466) (end 120.114466 73.839466) (width 1) (layer "F.Cu") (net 4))
 (segment (start 121.784466 108.284466) (end 123.354466 108.284466) (width 1) (layer "F.Cu") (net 4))
 (segment (start 120.72 110.03) (end 122.465534 108.284466) (width 1) (layer "B.Cu") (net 4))
 (segment (start 122.465534 108.284466) (end 123.354466 108.284466) (width 1) (layer "B.Cu") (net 4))
 (segment (start 118.6425 110.03) (end 120.72 110.03) (width 1) (layer "B.Cu") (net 4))
 (segment (start 100.6 82.328932) (end 100.6 99.768932) (width 1) (layer "F.Cu") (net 10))
 (segment (start 100.924466 82.004466) (end 100.6 82.328932) (width 1) (layer "F.Cu") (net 10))
 (segment (start 100.6 99.768932) (end 100.584466 99.784466) (width 1) (layer "F.Cu") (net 10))
 (segment (start 100.584466 99.784466) (end 102.514466 99.784466) (width 1) (layer "F.Cu") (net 10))
 (segment (start 102.514466 82.004466) (end 100.924466 82.004466) (width 1) (layer "F.Cu") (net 10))
 (segment (start 102.514466 99.784466) (end 104.215534 99.784466) (width 1) (layer "B.Cu") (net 10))
 (segment (start 123.354466 100.664466) (end 128.773034 100.664466) (width 1) (layer "B.Cu") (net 10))
 (segment (start 104.215534 99.784466) (end 106 98) (width 1) (layer "B.Cu") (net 10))
 (segment (start 106 98) (end 120.69 98) (width 1) (layer "B.Cu") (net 10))
 (segment (start 128.773034 100.664466) (end 129.25 100.1875) (width 1) (layer "B.Cu") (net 10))
 (segment (start 120.69 98) (end 123.354466 100.664466) (width 1) (layer "B.Cu") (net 10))
 (segment (start 106 92.4) (end 109.8 96.2) (width 1) (layer "F.Cu") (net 14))
 (segment (start 111.8 96.2) (end 115 99.4) (width 1) (layer "F.Cu") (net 14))
 (segment (start 109.8 96.2) (end 111.8 96.2) (width 1) (layer "F.Cu") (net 14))
 (segment (start 115 111.558932) (end 108.114466 118.444466) (width 1) (layer "F.Cu") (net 14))
 (segment (start 115 99.4) (end 115 111.558932) (width 1) (layer "F.Cu") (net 14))
 (segment (start 106 89.8) (end 106 92.4) (width 1) (layer "F.Cu") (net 14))
 (via (at 106 89.8) (size 1.6) (drill 1) (layers "F.Cu" "B.Cu") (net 14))
 (segment (start 118.4 70) (end 120.125534 68.274466) (width 1) (layer "B.Cu") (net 14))
 (segment (start 106 89.8) (end 111.2 89.8) (width 1) (layer "B.Cu") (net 14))
 (segment (start 120.125534 68.274466) (end 123.139466 68.274466) (width 1) (layer "B.Cu") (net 14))
 (segment (start 118.4 82.6) (end 118.4 70) (width 1) (layer "B.Cu") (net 14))
 (segment (start 111.2 89.8) (end 118.4 82.6) (width 1) (layer "B.Cu") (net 14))
 (segment (start 110.6 121.3) (end 110.284466 120.984466) (width 1) (layer "B.Cu") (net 5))
 (segment (start 153.8 100.2) (end 154.8 101.2) (width 1) (layer "B.Cu") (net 5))
 (segment (start 145.6 100.2) (end 153.8 100.2) (width 1) (layer "B.Cu") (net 5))
 (segment (start 152 121) (end 152 130.9) (width 1) (layer "B.Cu") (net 5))
 (segment (start 152 130.9) (end 144.3 138.6) (width 1) (layer "B.Cu") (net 5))
 (segment (start 154.8 101.2) (end 154.8 118.2) (width 1) (layer "B.Cu") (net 5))
 (segment (start 145.04 100.76) (end 145.6 100.2) (width 1) (layer "B.Cu") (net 5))
 (segment (start 110.284466 120.984466) (end 108.114466 120.984466) (width 1) (layer "B.Cu") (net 5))
 (segment (start 110.6 134) (end 110.6 121.3) (width 1) (layer "B.Cu") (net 5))
 (segment (start 154.8 118.2) (end 152 121) (width 1) (layer "B.Cu") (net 5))
 (segment (start 144.3 138.6) (end 115.2 138.6) (width 1) (layer "B.Cu") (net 5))
 (segment (start 145.04 102.25) (end 145.04 100.76) (width 1) (layer "B.Cu") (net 5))
 (segment (start 115.2 138.6) (end 110.6 134) (width 1) (layer "B.Cu") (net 5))
 (segment (start 120.8 59.4) (end 120.8 61.6) (width 1) (layer "F.Cu") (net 15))
 (segment (start 161.565 77.035) (end 162.8 75.8) (width 1) (layer "F.Cu") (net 15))
 (segment (start 121.4 58.8) (end 120.8 59.4) (width 1) (layer "F.Cu") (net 15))
 (segment (start 161.025 77.035) (end 161.565 77.035) (width 1) (layer "F.Cu") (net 15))
 (segment (start 148.4 58.8) (end 121.4 58.8) (width 1) (layer "F.Cu") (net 15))
 (segment (start 162.8 73.2) (end 148.4 58.8) (width 1) (layer "F.Cu") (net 15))
 (segment (start 162.8 75.8) (end 162.8 73.2) (width 1) (layer "F.Cu") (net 15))
 (segment (start 120.8 61.6) (end 122.394466 63.194466) (width 1) (layer "F.Cu") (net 15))
 (segment (start 122.394466 63.194466) (end 123.139466 63.194466) (width 1) (layer "F.Cu") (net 15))
 (segment (start 157.475 77.035) (end 155.035 77.035) (width 1) (layer "F.Cu") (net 16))
 (segment (start 155.035 77.035) (end 138.654466 60.654466) (width 1) (layer "F.Cu") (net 16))
 (segment (start 138.654466 60.654466) (end 123.139466 60.654466) (width 1) (layer "F.Cu") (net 16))
 (segment (start 131.935 135.865978) (end 133.200978 134.6) (width 1) (layer "B.Cu") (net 2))
 (segment (start 141.7 134.6) (end 150.12 126.18) (width 1) (layer "B.Cu") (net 2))
 (segment (start 131.935 136.425) (end 131.935 135.865978) (width 1) (layer "B.Cu") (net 2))
 (segment (start 150.12 126.18) (end 150.12 102.25) (width 1) (layer "B.Cu") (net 2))
 (segment (start 133.200978 134.6) (end 141.7 134.6) (width 1) (layer "B.Cu") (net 2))
 (segment (start 146.31 108.6) (end 152.66 102.25) (width 1) (layer "F.Cu") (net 7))
 (segment (start 131.935 132.875) (end 130.940148 131.880148) (width 1) (layer "F.Cu") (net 7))
 (segment (start 130.940148 121.409852) (end 143.75 108.6) (width 1) (layer "F.Cu") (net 7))
 (segment (start 130.940148 131.880148) (end 130.940148 121.409852) (width 1) (layer "F.Cu") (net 7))
 (segment (start 143.75 108.6) (end 146.31 108.6) (width 1) (layer "F.Cu") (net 7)))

